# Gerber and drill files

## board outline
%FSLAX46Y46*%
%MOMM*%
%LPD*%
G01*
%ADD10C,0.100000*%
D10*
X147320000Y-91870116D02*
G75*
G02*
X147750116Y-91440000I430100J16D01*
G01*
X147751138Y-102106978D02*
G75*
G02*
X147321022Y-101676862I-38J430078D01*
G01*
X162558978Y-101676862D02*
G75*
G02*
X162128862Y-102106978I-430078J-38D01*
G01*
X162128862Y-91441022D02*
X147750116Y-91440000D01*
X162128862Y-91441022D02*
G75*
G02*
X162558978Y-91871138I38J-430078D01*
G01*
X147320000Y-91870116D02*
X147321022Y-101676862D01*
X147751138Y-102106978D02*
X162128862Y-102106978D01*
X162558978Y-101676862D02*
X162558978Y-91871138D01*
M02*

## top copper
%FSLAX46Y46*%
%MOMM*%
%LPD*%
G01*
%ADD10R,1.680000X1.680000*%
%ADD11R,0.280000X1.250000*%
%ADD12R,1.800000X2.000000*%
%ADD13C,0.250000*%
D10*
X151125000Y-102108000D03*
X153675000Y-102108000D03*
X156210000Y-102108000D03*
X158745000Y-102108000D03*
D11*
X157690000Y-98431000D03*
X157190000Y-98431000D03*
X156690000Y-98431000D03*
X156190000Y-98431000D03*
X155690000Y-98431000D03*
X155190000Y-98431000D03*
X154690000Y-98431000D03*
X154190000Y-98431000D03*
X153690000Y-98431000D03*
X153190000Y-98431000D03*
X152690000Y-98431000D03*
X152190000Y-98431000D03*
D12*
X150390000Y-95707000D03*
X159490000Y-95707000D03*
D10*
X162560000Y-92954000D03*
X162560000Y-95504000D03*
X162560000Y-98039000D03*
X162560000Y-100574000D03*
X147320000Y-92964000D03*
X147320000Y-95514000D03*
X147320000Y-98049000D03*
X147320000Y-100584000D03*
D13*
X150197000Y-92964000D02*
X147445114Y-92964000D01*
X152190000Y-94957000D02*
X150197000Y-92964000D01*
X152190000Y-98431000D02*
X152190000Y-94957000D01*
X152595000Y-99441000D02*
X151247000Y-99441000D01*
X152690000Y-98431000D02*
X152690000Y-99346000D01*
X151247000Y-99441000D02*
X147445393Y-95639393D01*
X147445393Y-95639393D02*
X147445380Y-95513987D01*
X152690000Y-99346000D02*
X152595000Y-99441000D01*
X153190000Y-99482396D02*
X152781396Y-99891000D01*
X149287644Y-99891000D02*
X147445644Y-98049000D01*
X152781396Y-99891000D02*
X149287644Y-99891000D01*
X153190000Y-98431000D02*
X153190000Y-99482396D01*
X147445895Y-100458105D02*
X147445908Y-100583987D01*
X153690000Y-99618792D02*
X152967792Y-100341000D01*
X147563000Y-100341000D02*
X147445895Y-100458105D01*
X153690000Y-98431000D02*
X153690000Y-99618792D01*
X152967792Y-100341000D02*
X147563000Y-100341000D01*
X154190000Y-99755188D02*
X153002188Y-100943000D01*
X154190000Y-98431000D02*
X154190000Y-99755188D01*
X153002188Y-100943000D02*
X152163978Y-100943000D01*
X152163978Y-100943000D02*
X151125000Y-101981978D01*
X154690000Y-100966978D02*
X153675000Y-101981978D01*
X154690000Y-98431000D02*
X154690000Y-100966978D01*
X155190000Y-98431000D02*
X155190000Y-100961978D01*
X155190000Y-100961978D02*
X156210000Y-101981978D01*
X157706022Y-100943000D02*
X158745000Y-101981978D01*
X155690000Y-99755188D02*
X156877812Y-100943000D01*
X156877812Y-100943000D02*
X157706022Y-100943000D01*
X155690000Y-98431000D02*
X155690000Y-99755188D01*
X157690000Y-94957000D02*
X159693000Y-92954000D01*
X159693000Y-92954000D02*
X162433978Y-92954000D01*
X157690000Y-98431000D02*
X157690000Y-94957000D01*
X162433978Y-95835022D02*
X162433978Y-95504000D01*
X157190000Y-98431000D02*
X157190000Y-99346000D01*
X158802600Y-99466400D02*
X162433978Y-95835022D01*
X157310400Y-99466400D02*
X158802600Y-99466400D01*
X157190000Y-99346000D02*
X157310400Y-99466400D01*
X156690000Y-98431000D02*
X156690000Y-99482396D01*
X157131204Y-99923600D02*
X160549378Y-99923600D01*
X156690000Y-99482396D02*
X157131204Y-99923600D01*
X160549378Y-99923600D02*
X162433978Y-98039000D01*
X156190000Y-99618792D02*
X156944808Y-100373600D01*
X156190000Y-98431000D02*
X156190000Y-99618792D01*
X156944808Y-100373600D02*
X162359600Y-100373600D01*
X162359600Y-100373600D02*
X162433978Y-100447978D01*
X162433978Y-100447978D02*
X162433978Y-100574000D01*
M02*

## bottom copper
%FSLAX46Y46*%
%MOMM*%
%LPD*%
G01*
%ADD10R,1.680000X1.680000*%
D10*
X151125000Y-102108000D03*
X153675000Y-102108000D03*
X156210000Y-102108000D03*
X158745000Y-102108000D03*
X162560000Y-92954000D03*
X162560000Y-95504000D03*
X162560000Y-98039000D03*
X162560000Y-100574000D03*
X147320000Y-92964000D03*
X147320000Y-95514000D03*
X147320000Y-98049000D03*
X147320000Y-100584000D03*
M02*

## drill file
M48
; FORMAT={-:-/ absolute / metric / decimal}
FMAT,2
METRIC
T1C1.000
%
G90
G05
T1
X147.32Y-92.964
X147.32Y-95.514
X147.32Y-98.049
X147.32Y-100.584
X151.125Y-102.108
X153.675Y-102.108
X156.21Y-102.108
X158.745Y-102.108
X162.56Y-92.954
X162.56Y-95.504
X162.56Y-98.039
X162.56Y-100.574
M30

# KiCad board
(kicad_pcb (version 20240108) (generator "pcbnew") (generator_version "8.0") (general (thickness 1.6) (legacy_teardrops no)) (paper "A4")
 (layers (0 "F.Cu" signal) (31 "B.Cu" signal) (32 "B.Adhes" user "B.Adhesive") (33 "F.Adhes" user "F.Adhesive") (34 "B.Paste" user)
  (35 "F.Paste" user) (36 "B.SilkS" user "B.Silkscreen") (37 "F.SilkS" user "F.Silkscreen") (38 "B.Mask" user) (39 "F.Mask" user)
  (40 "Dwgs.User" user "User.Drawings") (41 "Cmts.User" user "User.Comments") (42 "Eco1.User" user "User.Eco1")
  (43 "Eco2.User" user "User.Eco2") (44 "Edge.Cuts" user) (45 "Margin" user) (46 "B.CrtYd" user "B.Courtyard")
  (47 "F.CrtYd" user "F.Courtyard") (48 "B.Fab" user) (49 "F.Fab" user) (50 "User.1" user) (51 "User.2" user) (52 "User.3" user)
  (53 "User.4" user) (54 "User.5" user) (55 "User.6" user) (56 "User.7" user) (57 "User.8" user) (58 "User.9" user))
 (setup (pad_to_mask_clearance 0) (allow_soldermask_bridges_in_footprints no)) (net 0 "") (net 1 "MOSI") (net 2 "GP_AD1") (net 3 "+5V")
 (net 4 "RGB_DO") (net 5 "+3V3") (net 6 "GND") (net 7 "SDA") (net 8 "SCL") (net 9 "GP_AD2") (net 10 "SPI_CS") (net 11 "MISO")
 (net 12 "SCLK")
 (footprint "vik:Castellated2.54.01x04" (layer "F.Cu") (at 162.555 102.658 90)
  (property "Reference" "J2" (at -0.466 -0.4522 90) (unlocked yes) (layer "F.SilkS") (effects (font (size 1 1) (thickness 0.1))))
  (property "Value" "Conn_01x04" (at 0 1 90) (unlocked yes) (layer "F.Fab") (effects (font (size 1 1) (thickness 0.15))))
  (pad "1" thru_hole rect (at 0.55 -11.43 90) (size 1.68 1.68) (drill 1) (layers "*.Cu" "*.Mask") (remove_unused_layers no) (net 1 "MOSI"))
  (pad "2" thru_hole rect (at 0.55 -8.88 90) (size 1.68 1.68) (drill 1) (layers "*.Cu" "*.Mask") (remove_unused_layers no) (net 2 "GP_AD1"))
  (pad "3" thru_hole rect (at 0.55 -6.345 90) (size 1.68 1.68) (drill 1) (layers "*.Cu" "*.Mask") (remove_unused_layers no) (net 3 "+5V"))
  (pad "4" thru_hole rect (at 0.55 -3.81 90) (size 1.68 1.68) (drill 1) (layers "*.Cu" "*.Mask") (remove_unused_layers no) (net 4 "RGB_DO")))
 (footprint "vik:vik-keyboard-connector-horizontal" (layer "F.Cu") (at 154.94 96.393 180)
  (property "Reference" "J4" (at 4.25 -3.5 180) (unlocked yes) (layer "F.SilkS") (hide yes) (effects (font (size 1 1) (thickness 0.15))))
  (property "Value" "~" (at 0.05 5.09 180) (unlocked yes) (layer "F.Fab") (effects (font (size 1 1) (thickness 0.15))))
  (pad "1" smd rect (at -2.75 -2.038 180) (size 0.28 1.25) (layers "F.Cu" "F.Paste" "F.Mask") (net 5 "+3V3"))
  (pad "2" smd rect (at -2.25 -2.038 180) (size 0.28 1.25) (layers "F.Cu" "F.Paste" "F.Mask") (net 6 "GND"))
  (pad "3" smd rect (at -1.75 -2.038 180) (size 0.28 1.25) (layers "F.Cu" "F.Paste" "F.Mask") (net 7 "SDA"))
  (pad "4" smd rect (at -1.25 -2.038 180) (size 0.28 1.25) (layers "F.Cu" "F.Paste" "F.Mask") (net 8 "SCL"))
  (pad "5" smd rect (at -0.75 -2.038 180) (size 0.28 1.25) (layers "F.Cu" "F.Paste" "F.Mask") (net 4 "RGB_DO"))
  (pad "6" smd rect (at -0.25 -2.038 180) (size 0.28 1.25) (layers "F.Cu" "F.Paste" "F.Mask") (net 3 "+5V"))
  (pad "7" smd rect (at 0.25 -2.038 180) (size 0.28 1.25) (layers "F.Cu" "F.Paste" "F.Mask") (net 2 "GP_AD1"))
  (pad "8" smd rect (at 0.75 -2.038 180) (size 0.28 1.25) (layers "F.Cu" "F.Paste" "F.Mask") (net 1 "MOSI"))
  (pad "9" smd rect (at 1.25 -2.038 180) (size 0.28 1.25) (layers "F.Cu" "F.Paste" "F.Mask") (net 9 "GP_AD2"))
  (pad "10" smd rect (at 1.75 -2.038 180) (size 0.28 1.25) (layers "F.Cu" "F.Paste" "F.Mask") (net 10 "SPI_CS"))
  (pad "11" smd rect (at 2.25 -2.038 180) (size 0.28 1.25) (layers "F.Cu" "F.Paste" "F.Mask") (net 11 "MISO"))
  (pad "12" smd rect (at 2.75 -2.038 180) (size 0.28 1.25) (layers "F.Cu" "F.Paste" "F.Mask") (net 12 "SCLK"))
  (pad "13" smd rect (at 4.55 0.686 180) (size 1.8 2) (layers "F.Cu" "F.Paste" "F.Mask"))
  (pad "14" smd rect (at -4.55 0.686 180) (size 1.8 2) (layers "F.Cu" "F.Paste" "F.Mask")))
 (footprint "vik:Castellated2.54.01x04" (layer "F.Cu") (at 162.01 104.384)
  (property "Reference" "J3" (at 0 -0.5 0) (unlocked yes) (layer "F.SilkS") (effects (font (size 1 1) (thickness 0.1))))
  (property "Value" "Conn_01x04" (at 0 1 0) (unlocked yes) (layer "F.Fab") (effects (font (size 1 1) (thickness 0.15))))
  (pad "1" thru_hole rect (at 0.55 -11.43) (size 1.68 1.68) (drill 1) (layers "*.Cu" "*.Mask") (remove_unused_layers no) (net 5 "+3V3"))
  (pad "2" thru_hole rect (at 0.55 -8.88) (size 1.68 1.68) (drill 1) (layers "*.Cu" "*.Mask") (remove_unused_layers no) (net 6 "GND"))
  (pad "3" thru_hole rect (at 0.55 -6.345) (size 1.68 1.68) (drill 1) (layers "*.Cu" "*.Mask") (remove_unused_layers no) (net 7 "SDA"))
  (pad "4" thru_hole rect (at 0.55 -3.81) (size 1.68 1.68) (drill 1) (layers "*.Cu" "*.Mask") (remove_unused_layers no) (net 8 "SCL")))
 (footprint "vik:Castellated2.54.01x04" (layer "F.Cu") (at 146.77 104.394)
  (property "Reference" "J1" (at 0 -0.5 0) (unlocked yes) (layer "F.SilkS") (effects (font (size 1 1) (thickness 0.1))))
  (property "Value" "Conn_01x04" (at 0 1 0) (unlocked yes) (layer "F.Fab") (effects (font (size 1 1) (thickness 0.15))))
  (pad "1" thru_hole rect (at 0.55 -11.43) (size 1.68 1.68) (drill 1) (layers "*.Cu" "*.Mask") (remove_unused_layers no) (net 12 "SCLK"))
  (pad "2" thru_hole rect (at 0.55 -8.88) (size 1.68 1.68) (drill 1) (layers "*.Cu" "*.Mask") (remove_unused_layers no) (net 11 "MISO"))
  (pad "3" thru_hole rect (at 0.55 -6.345) (size 1.68 1.68) (drill 1) (layers "*.Cu" "*.Mask") (remove_unused_layers no) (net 10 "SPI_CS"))
  (pad "4" thru_hole rect (at 0.55 -3.81) (size 1.68 1.68) (drill 1) (layers "*.Cu" "*.Mask") (remove_unused_layers no) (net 9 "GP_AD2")))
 (gr_arc (start 147.32 91.870116) (mid 147.445978 91.565978) (end 147.750116 91.44) (stroke (width 0.1) (type default)) (layer "Edge.Cuts"))
 (gr_arc (start 147.751138 102.106978) (mid 147.447 101.981) (end 147.321022 101.676862) (stroke (width 0.1) (type default))
  (layer "Edge.Cuts"))
 (gr_arc (start 162.558978 101.676862) (mid 162.433 101.981) (end 162.128862 102.106978) (stroke (width 0.1) (type default))
  (layer "Edge.Cuts"))
 (gr_line (start 162.128862 91.441022) (end 147.750116 91.44) (stroke (width 0.1) (type default)) (layer "Edge.Cuts"))
 (gr_arc (start 162.128862 91.441022) (mid 162.433 91.567) (end 162.558978 91.871138) (stroke (width 0.1) (type default))
  (layer "Edge.Cuts"))
 (gr_line (start 147.32 91.870116) (end 147.321022 101.676862) (stroke (width 0.1) (type default)) (layer "Edge.Cuts"))
 (gr_line (start 147.751138 102.106978) (end 162.128862 102.106978) (stroke (width 0.1) (type default)) (layer "Edge.Cuts"))
 (gr_line (start 162.558978 101.676862) (end 162.558978 91.871138) (stroke (width 0.1) (type default)) (layer "Edge.Cuts"))
 (segment (start 150.197 92.964) (end 147.445114 92.964) (width 0.25) (layer "F.Cu") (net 12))
 (segment (start 152.19 94.957) (end 150.197 92.964) (width 0.25) (layer "F.Cu") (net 12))
 (segment (start 152.19 98.431) (end 152.19 94.957) (width 0.25) (layer "F.Cu") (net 12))
 (segment (start 152.595 99.441) (end 151.247 99.441) (width 0.25) (layer "F.Cu") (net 11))
 (segment (start 152.69 98.431) (end 152.69 99.346) (width 0.25) (layer "F.Cu") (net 11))
 (segment (start 151.247 99.441) (end 147.445393 95.639393) (width 0.25) (layer "F.Cu") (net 11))
 (segment (start 147.445393 95.639393) (end 147.44538 95.513987) (width 0.25) (layer "F.Cu") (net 11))
 (segment (start 152.69 99.346) (end 152.595 99.441) (width 0.25) (layer "F.Cu") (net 11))
 (segment (start 153.19 99.482396) (end 152.781396 99.891) (width 0.25) (layer "F.Cu") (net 10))
 (segment (start 149.287644 99.891) (end 147.445644 98.049) (width 0.25) (layer "F.Cu") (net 10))
 (segment (start 152.781396 99.891) (end 149.287644 99.891) (width 0.25) (layer "F.Cu") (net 10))
 (segment (start 153.19 98.431) (end 153.19 99.482396) (width 0.25) (layer "F.Cu") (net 10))
 (segment (start 147.445895 100.458105) (end 147.445908 100.583987) (width 0.25) (layer "F.Cu") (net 9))
 (segment (start 153.69 99.618792) (end 152.967792 100.341) (width 0.25) (layer "F.Cu") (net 9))
 (segment (start 147.563 100.341) (end 147.445895 100.458105) (width 0.25) (layer "F.Cu") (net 9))
 (segment (start 153.69 98.431) (end 153.69 99.618792) (width 0.25) (layer "F.Cu") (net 9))
 (segment (start 152.967792 100.341) (end 147.563 100.341) (width 0.25) (layer "F.Cu") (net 9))
 (segment (start 154.19 99.755188) (end 153.002188 100.943) (width 0.25) (layer "F.Cu") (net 1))
 (segment (start 154.19 98.431) (end 154.19 99.755188) (width 0.25) (layer "F.Cu") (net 1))
 (segment (start 153.002188 100.943) (end 152.163978 100.943) (width 0.25) (layer "F.Cu") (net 1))
 (segment (start 152.163978 100.943) (end 151.125 101.981978) (width 0.25) (layer "F.Cu") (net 1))
 (segment (start 154.69 100.966978) (end 153.675 101.981978) (width 0.25) (layer "F.Cu") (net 2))
 (segment (start 154.69 98.431) (end 154.69 100.966978) (width 0.25) (layer "F.Cu") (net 2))
 (segment (start 155.19 98.431) (end 155.19 100.961978) (width 0.25) (layer "F.Cu") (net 3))
 (segment (start 155.19 100.961978) (end 156.21 101.981978) (width 0.25) (layer "F.Cu") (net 3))
 (segment (start 157.706022 100.943) (end 158.745 101.981978) (width 0.25) (layer "F.Cu") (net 4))
 (segment (start 155.69 99.755188) (end 156.877812 100.943) (width 0.25) (layer "F.Cu") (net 4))
 (segment (start 156.877812 100.943) (end 157.706022 100.943) (width 0.25) (layer "F.Cu") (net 4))
 (segment (start 155.69 98.431) (end 155.69 99.755188) (width 0.25) (layer "F.Cu") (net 4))
 (segment (start 157.69 94.957) (end 159.693 92.954) (width 0.25) (layer "F.Cu") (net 5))
 (segment (start 159.693 92.954) (end 162.433978 92.954) (width 0.25) (layer "F.Cu") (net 5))
 (segment (start 157.69 98.431) (end 157.69 94.957) (width 0.25) (layer "F.Cu") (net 5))
 (segment (start 162.433978 95.835022) (end 162.433978 95.504) (width 0.25) (layer "F.Cu") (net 6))
 (segment (start 157.19 98.431) (end 157.19 99.346) (width 0.25) (layer "F.Cu") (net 6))
 (segment (start 158.8026 99.4664) (end 162.433978 95.835022) (width 0.25) (layer "F.Cu") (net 6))
 (segment (start 157.3104 99.4664) (end 158.8026 99.4664) (width 0.25) (layer "F.Cu") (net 6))
 (segment (start 157.19 99.346) (end 157.3104 99.4664) (width 0.25) (layer "F.Cu") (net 6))
 (segment (start 156.69 98.431) (end 156.69 99.482396) (width 0.25) (layer "F.Cu") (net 7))
 (segment (start 157.131204 99.9236) (end 160.549378 99.9236) (width 0.25) (layer "F.Cu") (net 7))
 (segment (start 156.69 99.482396) (end 157.131204 99.9236) (width 0.25) (layer "F.Cu") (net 7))
 (segment (start 160.549378 99.9236) (end 162.433978 98.039) (width 0.25) (layer "F.Cu") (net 7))
 (segment (start 156.19 99.618792) (end 156.944808 100.3736) (width 0.25) (layer "F.Cu") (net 8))
 (segment (start 156.19 98.431) (end 156.19 99.618792) (width 0.25) (layer "F.Cu") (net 8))
 (segment (start 156.944808 100.3736) (end 162.3596 100.3736) (width 0.25) (layer "F.Cu") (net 8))
 (segment (start 162.3596 100.3736) (end 162.433978 100.447978) (width 0.25) (layer "F.Cu") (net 8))
 (segment (start 162.433978 100.447978) (end 162.433978 100.574) (width 0.25) (layer "F.Cu") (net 8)))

